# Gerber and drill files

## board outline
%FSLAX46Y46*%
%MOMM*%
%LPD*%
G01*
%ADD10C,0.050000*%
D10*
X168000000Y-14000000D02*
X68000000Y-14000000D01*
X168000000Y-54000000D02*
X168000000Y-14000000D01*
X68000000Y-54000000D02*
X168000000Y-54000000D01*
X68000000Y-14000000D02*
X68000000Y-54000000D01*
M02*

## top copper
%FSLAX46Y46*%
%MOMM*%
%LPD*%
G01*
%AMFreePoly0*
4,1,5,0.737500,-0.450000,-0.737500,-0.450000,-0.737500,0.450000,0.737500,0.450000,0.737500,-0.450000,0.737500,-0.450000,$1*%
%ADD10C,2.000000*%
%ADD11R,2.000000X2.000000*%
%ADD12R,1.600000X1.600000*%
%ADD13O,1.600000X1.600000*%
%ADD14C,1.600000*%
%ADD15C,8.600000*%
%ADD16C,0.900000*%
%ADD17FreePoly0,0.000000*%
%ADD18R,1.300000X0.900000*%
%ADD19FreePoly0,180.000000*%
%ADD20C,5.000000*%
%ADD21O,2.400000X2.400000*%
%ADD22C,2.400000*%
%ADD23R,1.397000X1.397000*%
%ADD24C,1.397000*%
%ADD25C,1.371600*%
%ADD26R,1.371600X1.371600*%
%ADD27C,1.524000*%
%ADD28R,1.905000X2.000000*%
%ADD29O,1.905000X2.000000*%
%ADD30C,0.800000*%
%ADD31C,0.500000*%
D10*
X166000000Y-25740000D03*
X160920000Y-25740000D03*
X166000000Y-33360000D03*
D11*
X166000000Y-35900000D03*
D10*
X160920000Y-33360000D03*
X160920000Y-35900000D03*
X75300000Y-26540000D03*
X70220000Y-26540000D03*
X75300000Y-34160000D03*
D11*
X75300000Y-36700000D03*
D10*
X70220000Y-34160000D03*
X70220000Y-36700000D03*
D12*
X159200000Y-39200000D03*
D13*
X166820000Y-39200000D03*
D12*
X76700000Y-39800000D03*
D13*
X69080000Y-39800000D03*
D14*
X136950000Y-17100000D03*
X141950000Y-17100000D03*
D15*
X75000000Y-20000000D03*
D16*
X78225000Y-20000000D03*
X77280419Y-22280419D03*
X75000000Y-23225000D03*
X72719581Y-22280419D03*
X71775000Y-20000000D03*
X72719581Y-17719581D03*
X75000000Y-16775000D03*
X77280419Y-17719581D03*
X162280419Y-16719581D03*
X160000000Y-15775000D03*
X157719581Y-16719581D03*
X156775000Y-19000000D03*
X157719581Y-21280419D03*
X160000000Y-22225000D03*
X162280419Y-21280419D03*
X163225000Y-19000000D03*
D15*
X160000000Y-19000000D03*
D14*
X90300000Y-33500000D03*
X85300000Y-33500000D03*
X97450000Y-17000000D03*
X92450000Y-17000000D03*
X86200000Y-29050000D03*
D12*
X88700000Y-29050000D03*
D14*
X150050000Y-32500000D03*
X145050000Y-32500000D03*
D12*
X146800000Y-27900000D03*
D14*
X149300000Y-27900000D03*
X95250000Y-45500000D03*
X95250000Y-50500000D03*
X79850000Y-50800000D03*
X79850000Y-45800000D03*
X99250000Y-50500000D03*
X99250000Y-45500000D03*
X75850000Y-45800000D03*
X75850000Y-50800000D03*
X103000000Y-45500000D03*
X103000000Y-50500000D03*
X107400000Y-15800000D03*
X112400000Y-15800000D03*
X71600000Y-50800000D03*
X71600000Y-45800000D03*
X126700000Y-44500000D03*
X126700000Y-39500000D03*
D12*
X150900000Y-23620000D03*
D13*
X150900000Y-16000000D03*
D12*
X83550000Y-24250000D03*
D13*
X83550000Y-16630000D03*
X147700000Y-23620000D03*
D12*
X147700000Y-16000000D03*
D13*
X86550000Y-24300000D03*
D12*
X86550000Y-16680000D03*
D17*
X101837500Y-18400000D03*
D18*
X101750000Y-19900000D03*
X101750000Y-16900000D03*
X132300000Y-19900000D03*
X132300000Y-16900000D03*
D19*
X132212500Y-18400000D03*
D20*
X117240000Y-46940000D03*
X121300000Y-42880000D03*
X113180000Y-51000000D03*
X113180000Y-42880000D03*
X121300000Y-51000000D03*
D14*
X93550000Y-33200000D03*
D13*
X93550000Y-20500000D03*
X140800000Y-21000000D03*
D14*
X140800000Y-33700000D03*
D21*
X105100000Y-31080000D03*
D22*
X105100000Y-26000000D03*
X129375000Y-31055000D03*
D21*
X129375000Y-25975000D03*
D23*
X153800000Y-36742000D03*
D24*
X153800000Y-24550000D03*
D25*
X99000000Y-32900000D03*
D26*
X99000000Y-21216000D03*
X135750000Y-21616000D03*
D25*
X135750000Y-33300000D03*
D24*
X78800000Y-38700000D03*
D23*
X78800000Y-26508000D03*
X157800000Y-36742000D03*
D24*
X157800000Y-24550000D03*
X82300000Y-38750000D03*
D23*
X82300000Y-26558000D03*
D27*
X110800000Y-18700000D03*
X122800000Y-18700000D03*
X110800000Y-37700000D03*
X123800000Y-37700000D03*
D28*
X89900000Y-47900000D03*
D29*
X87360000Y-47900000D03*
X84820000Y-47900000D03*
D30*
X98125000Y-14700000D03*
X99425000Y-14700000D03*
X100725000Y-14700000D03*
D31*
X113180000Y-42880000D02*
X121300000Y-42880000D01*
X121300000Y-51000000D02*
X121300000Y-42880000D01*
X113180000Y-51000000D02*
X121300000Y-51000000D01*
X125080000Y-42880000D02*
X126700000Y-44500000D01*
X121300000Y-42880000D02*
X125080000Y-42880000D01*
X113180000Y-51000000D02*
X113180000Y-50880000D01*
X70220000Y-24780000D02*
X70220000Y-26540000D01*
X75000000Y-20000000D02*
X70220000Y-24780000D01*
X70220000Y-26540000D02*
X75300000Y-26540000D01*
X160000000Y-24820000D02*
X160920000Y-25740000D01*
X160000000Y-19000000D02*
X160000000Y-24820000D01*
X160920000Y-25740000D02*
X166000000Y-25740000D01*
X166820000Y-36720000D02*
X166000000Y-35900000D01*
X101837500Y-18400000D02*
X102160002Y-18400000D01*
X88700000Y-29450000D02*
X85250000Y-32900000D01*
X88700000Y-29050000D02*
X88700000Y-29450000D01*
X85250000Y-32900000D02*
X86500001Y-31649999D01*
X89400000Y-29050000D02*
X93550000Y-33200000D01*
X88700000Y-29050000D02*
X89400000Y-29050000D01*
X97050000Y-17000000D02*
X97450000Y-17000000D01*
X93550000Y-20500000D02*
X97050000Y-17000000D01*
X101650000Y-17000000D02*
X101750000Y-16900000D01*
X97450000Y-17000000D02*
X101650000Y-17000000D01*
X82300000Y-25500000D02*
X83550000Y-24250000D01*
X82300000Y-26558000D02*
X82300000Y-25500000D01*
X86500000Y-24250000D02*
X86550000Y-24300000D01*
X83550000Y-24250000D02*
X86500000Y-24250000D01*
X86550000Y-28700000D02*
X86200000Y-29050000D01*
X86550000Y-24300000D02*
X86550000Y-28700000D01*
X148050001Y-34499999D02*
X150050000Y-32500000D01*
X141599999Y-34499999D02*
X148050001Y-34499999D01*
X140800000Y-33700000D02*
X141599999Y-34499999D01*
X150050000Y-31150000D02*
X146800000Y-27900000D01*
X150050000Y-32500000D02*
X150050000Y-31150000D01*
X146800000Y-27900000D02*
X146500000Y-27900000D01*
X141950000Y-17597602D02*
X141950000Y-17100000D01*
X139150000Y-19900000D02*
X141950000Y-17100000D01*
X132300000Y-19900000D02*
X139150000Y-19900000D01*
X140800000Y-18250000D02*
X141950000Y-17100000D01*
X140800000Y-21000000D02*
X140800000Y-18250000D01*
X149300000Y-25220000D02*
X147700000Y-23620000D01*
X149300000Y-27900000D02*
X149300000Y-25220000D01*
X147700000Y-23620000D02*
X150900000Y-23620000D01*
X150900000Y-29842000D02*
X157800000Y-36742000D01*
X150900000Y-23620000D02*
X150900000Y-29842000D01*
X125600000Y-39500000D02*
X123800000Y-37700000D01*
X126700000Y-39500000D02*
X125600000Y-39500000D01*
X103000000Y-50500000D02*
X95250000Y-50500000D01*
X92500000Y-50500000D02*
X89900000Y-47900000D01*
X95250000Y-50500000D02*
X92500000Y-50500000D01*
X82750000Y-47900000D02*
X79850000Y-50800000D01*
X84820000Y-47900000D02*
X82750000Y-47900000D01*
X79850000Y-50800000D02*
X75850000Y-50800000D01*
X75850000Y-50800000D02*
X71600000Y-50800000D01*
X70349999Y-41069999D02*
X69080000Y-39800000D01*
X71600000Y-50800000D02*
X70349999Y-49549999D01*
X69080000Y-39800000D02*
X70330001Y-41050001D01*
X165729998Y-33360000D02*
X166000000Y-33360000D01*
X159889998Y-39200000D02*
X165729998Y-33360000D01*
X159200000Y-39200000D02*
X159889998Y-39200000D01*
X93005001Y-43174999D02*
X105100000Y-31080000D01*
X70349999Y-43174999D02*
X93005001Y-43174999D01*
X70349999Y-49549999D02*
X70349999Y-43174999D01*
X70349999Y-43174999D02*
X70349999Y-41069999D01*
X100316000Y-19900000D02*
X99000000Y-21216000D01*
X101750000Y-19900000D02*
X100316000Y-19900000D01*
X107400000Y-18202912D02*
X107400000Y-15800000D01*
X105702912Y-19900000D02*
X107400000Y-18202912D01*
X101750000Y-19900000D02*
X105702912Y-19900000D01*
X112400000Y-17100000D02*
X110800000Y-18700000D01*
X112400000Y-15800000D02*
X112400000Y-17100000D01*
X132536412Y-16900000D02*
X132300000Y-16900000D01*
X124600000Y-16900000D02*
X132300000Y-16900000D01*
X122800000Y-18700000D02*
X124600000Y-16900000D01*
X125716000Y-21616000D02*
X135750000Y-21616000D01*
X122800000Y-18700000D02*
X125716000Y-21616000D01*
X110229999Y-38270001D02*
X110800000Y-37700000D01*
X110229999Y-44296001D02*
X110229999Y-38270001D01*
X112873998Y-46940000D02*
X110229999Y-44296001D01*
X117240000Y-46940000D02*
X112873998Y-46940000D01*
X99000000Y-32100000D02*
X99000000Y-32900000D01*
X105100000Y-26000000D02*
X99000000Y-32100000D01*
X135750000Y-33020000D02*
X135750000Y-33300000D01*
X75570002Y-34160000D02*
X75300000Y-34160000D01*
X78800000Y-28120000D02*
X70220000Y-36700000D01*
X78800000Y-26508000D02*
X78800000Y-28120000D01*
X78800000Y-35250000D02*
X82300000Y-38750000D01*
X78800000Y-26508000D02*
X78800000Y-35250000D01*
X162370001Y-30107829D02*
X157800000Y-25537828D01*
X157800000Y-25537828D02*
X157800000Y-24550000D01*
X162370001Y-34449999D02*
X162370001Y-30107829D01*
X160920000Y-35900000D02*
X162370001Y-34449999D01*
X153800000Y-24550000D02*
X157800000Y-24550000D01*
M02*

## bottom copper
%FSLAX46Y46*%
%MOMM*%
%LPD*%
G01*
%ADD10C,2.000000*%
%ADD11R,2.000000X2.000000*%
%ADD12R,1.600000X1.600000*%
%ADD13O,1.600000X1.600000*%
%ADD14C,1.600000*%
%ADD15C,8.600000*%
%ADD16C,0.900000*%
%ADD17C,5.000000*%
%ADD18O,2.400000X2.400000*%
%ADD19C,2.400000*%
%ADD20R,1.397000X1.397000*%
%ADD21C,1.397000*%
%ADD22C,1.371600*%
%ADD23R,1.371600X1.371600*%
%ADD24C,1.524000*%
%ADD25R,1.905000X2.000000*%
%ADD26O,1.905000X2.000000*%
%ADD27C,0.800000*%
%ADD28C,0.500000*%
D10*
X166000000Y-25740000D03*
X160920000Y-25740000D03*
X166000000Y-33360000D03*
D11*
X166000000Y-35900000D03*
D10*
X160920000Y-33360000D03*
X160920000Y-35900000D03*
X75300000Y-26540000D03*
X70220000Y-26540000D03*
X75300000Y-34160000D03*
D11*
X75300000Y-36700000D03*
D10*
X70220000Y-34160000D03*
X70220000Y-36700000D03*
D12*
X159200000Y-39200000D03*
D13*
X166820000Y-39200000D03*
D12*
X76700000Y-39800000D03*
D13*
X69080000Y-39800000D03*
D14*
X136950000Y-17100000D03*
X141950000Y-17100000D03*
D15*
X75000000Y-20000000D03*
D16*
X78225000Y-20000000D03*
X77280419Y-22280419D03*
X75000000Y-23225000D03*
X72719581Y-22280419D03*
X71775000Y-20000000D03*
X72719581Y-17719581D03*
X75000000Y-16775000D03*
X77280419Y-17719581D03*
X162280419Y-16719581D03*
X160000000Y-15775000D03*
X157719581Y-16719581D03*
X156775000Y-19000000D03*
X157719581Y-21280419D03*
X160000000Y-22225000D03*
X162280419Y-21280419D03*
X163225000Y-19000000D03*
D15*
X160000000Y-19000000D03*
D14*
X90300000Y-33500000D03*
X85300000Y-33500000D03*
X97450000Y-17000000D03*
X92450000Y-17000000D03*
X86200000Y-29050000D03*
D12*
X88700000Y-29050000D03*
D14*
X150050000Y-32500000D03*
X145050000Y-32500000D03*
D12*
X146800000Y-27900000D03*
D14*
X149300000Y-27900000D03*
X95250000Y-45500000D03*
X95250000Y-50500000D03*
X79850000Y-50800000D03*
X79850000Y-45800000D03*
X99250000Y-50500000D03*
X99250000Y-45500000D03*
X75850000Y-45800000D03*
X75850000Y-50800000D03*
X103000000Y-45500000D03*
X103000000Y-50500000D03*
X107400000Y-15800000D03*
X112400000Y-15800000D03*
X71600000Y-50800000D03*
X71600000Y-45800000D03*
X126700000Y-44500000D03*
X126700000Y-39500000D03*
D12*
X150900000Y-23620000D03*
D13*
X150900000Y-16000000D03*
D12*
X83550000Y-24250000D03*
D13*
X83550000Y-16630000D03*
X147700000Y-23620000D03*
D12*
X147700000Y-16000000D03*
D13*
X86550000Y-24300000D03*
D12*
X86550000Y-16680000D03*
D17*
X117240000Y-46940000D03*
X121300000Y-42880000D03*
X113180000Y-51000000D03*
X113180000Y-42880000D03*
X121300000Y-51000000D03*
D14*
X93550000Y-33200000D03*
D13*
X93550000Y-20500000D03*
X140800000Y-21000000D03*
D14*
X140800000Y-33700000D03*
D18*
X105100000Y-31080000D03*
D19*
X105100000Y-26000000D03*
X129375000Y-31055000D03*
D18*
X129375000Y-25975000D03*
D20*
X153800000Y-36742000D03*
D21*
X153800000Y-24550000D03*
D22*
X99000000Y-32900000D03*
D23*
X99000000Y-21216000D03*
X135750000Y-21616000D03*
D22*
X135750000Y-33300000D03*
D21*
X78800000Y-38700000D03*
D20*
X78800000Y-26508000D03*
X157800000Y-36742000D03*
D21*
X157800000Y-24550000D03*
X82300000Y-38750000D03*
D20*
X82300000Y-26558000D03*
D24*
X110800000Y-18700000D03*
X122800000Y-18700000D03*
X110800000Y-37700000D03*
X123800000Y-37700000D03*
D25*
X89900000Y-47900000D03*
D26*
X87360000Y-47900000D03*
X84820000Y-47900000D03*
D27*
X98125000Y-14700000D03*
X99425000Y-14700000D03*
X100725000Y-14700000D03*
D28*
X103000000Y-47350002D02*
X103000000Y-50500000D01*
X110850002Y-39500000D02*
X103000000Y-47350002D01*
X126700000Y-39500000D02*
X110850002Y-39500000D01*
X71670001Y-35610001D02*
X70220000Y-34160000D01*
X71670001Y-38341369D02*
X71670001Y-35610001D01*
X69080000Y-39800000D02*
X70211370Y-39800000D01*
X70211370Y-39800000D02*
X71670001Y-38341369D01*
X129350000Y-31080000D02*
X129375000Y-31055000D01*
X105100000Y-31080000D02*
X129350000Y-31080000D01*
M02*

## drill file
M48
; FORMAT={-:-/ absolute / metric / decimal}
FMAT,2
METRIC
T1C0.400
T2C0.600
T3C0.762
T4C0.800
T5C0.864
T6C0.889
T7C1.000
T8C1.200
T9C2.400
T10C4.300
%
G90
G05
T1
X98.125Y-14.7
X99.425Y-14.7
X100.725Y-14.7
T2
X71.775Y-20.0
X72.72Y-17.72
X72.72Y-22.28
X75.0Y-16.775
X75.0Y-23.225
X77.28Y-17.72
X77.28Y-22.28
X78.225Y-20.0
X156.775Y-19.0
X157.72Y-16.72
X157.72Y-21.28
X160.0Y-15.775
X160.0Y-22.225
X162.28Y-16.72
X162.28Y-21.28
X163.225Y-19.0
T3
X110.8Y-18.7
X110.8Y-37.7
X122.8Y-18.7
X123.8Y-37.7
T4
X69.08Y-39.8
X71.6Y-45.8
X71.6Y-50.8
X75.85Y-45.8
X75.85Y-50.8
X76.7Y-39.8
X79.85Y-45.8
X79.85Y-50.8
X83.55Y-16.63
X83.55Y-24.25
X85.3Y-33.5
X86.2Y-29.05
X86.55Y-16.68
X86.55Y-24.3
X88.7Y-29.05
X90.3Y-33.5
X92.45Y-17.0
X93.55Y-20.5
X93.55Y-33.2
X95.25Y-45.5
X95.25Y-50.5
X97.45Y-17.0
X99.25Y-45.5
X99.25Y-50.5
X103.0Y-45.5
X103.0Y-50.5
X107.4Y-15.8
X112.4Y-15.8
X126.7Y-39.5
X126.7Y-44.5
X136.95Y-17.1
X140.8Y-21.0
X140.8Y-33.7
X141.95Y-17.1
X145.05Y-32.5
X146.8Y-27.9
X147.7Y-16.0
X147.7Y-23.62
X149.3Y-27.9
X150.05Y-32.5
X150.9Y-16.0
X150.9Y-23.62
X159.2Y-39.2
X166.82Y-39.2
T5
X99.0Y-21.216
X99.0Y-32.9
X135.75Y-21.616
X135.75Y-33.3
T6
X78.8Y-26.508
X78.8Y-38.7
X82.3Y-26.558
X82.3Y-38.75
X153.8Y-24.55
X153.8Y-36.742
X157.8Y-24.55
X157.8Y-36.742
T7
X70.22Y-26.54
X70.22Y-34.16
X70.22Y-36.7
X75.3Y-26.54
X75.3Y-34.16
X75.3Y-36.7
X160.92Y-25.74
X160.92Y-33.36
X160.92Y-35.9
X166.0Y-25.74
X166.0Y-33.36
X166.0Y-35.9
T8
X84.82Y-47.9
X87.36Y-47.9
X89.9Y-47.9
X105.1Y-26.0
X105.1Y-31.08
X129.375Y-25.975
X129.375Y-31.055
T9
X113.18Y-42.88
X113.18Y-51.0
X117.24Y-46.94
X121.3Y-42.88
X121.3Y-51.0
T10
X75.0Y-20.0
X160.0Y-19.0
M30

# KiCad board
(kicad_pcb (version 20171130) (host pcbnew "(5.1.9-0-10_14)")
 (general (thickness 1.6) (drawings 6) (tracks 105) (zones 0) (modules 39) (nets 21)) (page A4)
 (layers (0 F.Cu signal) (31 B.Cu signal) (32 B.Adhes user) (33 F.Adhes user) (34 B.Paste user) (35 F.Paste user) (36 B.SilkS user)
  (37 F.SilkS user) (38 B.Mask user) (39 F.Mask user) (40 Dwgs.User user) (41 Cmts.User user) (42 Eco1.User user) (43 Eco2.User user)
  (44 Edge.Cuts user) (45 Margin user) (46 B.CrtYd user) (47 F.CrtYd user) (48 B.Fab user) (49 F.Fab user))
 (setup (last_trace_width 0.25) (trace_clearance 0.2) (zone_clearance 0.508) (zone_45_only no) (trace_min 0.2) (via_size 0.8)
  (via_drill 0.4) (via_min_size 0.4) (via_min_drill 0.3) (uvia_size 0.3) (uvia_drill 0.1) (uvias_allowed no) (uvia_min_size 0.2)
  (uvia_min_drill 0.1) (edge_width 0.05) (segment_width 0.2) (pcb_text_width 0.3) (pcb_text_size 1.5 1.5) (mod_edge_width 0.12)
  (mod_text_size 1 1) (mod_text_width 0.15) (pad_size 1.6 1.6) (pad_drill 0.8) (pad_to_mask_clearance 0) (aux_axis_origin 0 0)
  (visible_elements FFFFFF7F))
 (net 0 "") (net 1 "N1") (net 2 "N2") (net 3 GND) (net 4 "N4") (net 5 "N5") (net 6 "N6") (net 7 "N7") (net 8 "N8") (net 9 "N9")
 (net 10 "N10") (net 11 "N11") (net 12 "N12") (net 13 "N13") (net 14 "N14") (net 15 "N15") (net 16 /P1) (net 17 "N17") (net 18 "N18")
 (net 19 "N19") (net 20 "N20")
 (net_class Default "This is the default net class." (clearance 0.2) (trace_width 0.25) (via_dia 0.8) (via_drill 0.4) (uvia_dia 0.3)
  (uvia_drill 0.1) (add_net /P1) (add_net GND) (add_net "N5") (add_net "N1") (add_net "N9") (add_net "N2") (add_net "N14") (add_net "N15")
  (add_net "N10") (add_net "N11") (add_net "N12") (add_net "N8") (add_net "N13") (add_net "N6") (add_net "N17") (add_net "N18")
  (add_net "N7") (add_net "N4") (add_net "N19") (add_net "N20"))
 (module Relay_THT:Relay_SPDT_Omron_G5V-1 (layer F.Cu) (at 166 35.9 180)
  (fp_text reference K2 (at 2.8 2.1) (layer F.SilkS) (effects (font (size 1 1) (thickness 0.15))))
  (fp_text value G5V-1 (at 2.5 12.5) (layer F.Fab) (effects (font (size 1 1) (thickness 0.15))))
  (pad 5 thru_hole circle (at 0 10.16 180) (size 2 2) (drill 1) (layers *.Cu *.Mask) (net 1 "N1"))
  (pad 6 thru_hole circle (at 5.08 10.16 180) (size 2 2) (drill 1) (layers *.Cu *.Mask) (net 1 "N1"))
  (pad 2 thru_hole circle (at 0 2.54 180) (size 2 2) (drill 1) (layers *.Cu *.Mask) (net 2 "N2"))
  (pad 1 thru_hole rect (at 0 0 180) (size 2 2) (drill 1) (layers *.Cu *.Mask) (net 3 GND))
  (pad 9 thru_hole circle (at 5.08 2.54 180) (size 2 2) (drill 1) (layers *.Cu *.Mask) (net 3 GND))
  (pad 10 thru_hole circle (at 5.08 0 180) (size 2 2) (drill 1) (layers *.Cu *.Mask) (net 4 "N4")))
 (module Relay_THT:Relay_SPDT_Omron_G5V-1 (layer F.Cu) (at 75.3 36.7 180)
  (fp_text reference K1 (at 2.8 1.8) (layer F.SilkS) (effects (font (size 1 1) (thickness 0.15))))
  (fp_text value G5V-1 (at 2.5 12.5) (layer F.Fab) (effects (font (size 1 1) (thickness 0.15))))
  (pad 5 thru_hole circle (at 0 10.16 180) (size 2 2) (drill 1) (layers *.Cu *.Mask) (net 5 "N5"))
  (pad 6 thru_hole circle (at 5.08 10.16 180) (size 2 2) (drill 1) (layers *.Cu *.Mask) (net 5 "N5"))
  (pad 2 thru_hole circle (at 0 2.54 180) (size 2 2) (drill 1) (layers *.Cu *.Mask) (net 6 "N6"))
  (pad 1 thru_hole rect (at 0 0 180) (size 2 2) (drill 1) (layers *.Cu *.Mask) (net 3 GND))
  (pad 9 thru_hole circle (at 5.08 2.54 180) (size 2 2) (drill 1) (layers *.Cu *.Mask) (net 2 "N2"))
  (pad 10 thru_hole circle (at 5.08 0 180) (size 2 2) (drill 1) (layers *.Cu *.Mask) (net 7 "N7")))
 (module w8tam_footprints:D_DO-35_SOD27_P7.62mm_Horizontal (layer F.Cu) (at 159.2 39.2)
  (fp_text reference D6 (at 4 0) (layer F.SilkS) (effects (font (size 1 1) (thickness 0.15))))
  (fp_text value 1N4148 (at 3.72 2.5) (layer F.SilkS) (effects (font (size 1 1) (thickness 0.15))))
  (pad 1 thru_hole rect (at 0 0) (size 1.6 1.6) (drill 0.8) (layers *.Cu *.Mask) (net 2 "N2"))
  (pad 2 thru_hole oval (at 7.62 0) (size 1.6 1.6) (drill 0.8) (layers *.Cu *.Mask) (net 3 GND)))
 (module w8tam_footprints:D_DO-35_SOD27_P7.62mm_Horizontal (layer F.Cu) (at 76.7 39.8 180)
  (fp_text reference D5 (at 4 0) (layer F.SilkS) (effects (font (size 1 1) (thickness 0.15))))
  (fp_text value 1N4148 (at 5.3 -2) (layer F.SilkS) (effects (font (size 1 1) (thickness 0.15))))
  (pad 1 thru_hole rect (at 0 0 180) (size 1.6 1.6) (drill 0.8) (layers *.Cu *.Mask) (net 3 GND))
  (pad 2 thru_hole oval (at 7.62 0 180) (size 1.6 1.6) (drill 0.8) (layers *.Cu *.Mask) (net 2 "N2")))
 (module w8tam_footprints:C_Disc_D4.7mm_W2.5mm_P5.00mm (layer F.Cu) (at 141.95 17.1 180)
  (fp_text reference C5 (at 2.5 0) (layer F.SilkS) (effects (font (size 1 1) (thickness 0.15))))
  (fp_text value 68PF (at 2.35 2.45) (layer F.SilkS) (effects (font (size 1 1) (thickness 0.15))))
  (pad 2 thru_hole circle (at 5 0 180) (size 1.6 1.6) (drill 0.8) (layers *.Cu *.Mask) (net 3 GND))
  (pad 1 thru_hole circle (at 0 0 180) (size 1.6 1.6) (drill 0.8) (layers *.Cu *.Mask) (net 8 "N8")))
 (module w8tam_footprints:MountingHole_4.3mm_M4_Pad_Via (layer F.Cu) (at 75 20)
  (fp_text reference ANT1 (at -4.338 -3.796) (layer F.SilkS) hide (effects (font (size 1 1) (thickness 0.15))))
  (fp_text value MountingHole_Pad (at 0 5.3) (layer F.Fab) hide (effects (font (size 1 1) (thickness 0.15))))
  (pad 1 thru_hole circle (at 0 0) (size 8.6 8.6) (drill 4.3) (layers *.Cu *.Mask) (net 5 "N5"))
  (pad 1 thru_hole circle (at 3.225 0) (size 0.9 0.9) (drill 0.6) (layers *.Cu *.Mask) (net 5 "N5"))
  (pad 1 thru_hole circle (at 2.280419 2.280419) (size 0.9 0.9) (drill 0.6) (layers *.Cu *.Mask) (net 5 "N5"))
  (pad 1 thru_hole circle (at 0 3.225) (size 0.9 0.9) (drill 0.6) (layers *.Cu *.Mask) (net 5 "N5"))
  (pad 1 thru_hole circle (at -2.280419 2.280419) (size 0.9 0.9) (drill 0.6) (layers *.Cu *.Mask) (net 5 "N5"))
  (pad 1 thru_hole circle (at -3.225 0) (size 0.9 0.9) (drill 0.6) (layers *.Cu *.Mask) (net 5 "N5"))
  (pad 1 thru_hole circle (at -2.280419 -2.280419) (size 0.9 0.9) (drill 0.6) (layers *.Cu *.Mask) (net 5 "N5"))
  (pad 1 thru_hole circle (at 0 -3.225) (size 0.9 0.9) (drill 0.6) (layers *.Cu *.Mask) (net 5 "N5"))
  (pad 1 thru_hole circle (at 2.280419 -2.280419) (size 0.9 0.9) (drill 0.6) (layers *.Cu *.Mask) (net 5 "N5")))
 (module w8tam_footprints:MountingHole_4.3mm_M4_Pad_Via (layer F.Cu) (at 160 19)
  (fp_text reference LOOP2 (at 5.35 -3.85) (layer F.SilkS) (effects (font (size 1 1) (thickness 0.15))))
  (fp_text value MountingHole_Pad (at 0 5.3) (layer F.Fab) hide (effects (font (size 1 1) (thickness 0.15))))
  (pad 1 thru_hole circle (at 2.280419 -2.280419) (size 0.9 0.9) (drill 0.6) (layers *.Cu *.Mask) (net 1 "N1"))
  (pad 1 thru_hole circle (at 0 -3.225) (size 0.9 0.9) (drill 0.6) (layers *.Cu *.Mask) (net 1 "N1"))
  (pad 1 thru_hole circle (at -2.280419 -2.280419) (size 0.9 0.9) (drill 0.6) (layers *.Cu *.Mask) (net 1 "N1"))
  (pad 1 thru_hole circle (at -3.225 0) (size 0.9 0.9) (drill 0.6) (layers *.Cu *.Mask) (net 1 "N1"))
  (pad 1 thru_hole circle (at -2.280419 2.280419) (size 0.9 0.9) (drill 0.6) (layers *.Cu *.Mask) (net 1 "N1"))
  (pad 1 thru_hole circle (at 0 3.225) (size 0.9 0.9) (drill 0.6) (layers *.Cu *.Mask) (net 1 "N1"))
  (pad 1 thru_hole circle (at 2.280419 2.280419) (size 0.9 0.9) (drill 0.6) (layers *.Cu *.Mask) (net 1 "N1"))
  (pad 1 thru_hole circle (at 3.225 0) (size 0.9 0.9) (drill 0.6) (layers *.Cu *.Mask) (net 1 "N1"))
  (pad 1 thru_hole circle (at 0 0) (size 8.6 8.6) (drill 4.3) (layers *.Cu *.Mask) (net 1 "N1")))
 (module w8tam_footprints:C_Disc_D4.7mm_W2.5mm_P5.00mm (layer F.Cu) (at 85.3 33.5)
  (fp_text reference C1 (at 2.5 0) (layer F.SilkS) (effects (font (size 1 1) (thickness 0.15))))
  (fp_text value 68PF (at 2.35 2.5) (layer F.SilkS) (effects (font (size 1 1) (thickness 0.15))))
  (pad 2 thru_hole circle (at 5 0) (size 1.6 1.6) (drill 0.8) (layers *.Cu *.Mask) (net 3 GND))
  (pad 1 thru_hole circle (at 0 0) (size 1.6 1.6) (drill 0.8) (layers *.Cu *.Mask) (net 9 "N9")))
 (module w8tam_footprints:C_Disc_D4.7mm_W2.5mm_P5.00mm (layer F.Cu) (at 97.45 17 180)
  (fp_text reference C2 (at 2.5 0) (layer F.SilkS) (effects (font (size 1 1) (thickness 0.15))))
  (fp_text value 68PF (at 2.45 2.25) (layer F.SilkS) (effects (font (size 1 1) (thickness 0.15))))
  (pad 1 thru_hole circle (at 0 0 180) (size 1.6 1.6) (drill 0.8) (layers *.Cu *.Mask) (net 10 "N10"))
  (pad 2 thru_hole circle (at 5 0 180) (size 1.6 1.6) (drill 0.8) (layers *.Cu *.Mask) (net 3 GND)))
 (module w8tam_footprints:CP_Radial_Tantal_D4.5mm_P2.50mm (layer F.Cu) (at 88.7 29.05 180)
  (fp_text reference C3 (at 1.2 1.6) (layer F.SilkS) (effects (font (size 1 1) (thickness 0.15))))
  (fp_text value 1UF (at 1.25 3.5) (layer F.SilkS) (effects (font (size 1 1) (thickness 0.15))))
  (pad 2 thru_hole circle (at 2.5 0 180) (size 1.6 1.6) (drill 0.8) (layers *.Cu *.Mask) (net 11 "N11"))
  (pad 1 thru_hole rect (at 0 0 180) (size 1.6 1.6) (drill 0.8) (layers *.Cu *.Mask) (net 9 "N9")))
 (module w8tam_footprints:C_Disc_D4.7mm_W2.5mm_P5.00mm (layer F.Cu) (at 150.05 32.5 180)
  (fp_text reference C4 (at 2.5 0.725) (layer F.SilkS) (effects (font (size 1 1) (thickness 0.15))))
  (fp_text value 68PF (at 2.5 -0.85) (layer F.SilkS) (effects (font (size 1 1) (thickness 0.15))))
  (pad 1 thru_hole circle (at 0 0 180) (size 1.6 1.6) (drill 0.8) (layers *.Cu *.Mask) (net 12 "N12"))
  (pad 2 thru_hole circle (at 5 0 180) (size 1.6 1.6) (drill 0.8) (layers *.Cu *.Mask) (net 3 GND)))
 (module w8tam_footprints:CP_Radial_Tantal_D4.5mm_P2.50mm (layer F.Cu) (at 146.8 27.9)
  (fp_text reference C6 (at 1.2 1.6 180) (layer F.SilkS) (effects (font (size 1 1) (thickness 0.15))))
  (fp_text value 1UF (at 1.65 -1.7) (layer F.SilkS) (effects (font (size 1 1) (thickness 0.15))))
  (pad 1 thru_hole rect (at 0 0) (size 1.6 1.6) (drill 0.8) (layers *.Cu *.Mask) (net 12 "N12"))
  (pad 2 thru_hole circle (at 2.5 0) (size 1.6 1.6) (drill 0.8) (layers *.Cu *.Mask) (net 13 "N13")))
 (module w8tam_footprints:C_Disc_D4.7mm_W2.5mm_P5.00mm (layer F.Cu) (at 95.25 50.5 90)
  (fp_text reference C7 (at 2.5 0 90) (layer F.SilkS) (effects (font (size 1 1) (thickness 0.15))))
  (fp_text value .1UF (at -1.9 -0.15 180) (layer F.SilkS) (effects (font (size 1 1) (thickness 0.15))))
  (pad 2 thru_hole circle (at 5 0 90) (size 1.6 1.6) (drill 0.8) (layers *.Cu *.Mask) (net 3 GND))
  (pad 1 thru_hole circle (at 0 0 90) (size 1.6 1.6) (drill 0.8) (layers *.Cu *.Mask) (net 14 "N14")))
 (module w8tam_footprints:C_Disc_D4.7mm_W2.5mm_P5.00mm (layer F.Cu) (at 79.85 50.8 90)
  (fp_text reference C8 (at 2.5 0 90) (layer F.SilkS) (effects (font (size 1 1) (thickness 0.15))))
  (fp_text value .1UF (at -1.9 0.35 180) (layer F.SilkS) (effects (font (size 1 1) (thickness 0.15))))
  (pad 1 thru_hole circle (at 0 0 90) (size 1.6 1.6) (drill 0.8) (layers *.Cu *.Mask) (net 2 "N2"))
  (pad 2 thru_hole circle (at 5 0 90) (size 1.6 1.6) (drill 0.8) (layers *.Cu *.Mask) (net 3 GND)))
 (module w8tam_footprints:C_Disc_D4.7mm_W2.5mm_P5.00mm (layer F.Cu) (at 99.25 50.5 90)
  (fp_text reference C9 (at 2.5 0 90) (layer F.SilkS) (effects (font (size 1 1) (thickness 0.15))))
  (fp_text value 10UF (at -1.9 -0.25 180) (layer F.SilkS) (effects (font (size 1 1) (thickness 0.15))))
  (pad 1 thru_hole circle (at 0 0 90) (size 1.6 1.6) (drill 0.8) (layers *.Cu *.Mask) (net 14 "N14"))
  (pad 2 thru_hole circle (at 5 0 90) (size 1.6 1.6) (drill 0.8) (layers *.Cu *.Mask) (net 3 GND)))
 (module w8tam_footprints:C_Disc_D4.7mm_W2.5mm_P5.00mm (layer F.Cu) (at 75.85 50.8 90)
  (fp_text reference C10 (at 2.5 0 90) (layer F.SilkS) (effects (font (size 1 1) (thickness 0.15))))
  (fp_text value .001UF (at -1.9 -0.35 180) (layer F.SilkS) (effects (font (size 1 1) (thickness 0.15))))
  (pad 2 thru_hole circle (at 5 0 90) (size 1.6 1.6) (drill 0.8) (layers *.Cu *.Mask) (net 3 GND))
  (pad 1 thru_hole circle (at 0 0 90) (size 1.6 1.6) (drill 0.8) (layers *.Cu *.Mask) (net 2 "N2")))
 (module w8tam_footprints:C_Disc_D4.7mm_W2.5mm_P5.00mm (layer F.Cu) (at 103 50.5 90)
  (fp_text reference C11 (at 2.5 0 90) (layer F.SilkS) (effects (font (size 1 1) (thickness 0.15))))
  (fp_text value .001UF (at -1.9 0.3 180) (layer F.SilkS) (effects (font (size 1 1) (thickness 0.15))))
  (pad 2 thru_hole circle (at 5 0 90) (size 1.6 1.6) (drill 0.8) (layers *.Cu *.Mask) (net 3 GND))
  (pad 1 thru_hole circle (at 0 0 90) (size 1.6 1.6) (drill 0.8) (layers *.Cu *.Mask) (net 14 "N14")))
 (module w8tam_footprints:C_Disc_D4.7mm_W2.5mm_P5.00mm (layer F.Cu) (at 112.4 15.8 180)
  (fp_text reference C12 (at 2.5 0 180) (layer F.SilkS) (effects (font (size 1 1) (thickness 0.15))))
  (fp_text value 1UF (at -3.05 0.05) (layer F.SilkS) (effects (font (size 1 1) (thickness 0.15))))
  (pad 2 thru_hole circle (at 5 0 180) (size 1.6 1.6) (drill 0.8) (layers *.Cu *.Mask) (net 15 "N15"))
  (pad 1 thru_hole circle (at 0 0 180) (size 1.6 1.6) (drill 0.8) (layers *.Cu *.Mask) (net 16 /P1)))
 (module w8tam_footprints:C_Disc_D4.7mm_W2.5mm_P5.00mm (layer F.Cu) (at 71.6 50.8 90)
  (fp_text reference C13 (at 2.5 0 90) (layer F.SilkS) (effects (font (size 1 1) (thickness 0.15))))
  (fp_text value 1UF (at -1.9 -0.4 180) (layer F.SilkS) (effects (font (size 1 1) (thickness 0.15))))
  (pad 1 thru_hole circle (at 0 0 90) (size 1.6 1.6) (drill 0.8) (layers *.Cu *.Mask) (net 2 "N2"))
  (pad 2 thru_hole circle (at 5 0 90) (size 1.6 1.6) (drill 0.8) (layers *.Cu *.Mask) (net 3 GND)))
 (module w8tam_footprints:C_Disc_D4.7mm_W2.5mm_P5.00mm (layer F.Cu) (at 126.7 44.5 90)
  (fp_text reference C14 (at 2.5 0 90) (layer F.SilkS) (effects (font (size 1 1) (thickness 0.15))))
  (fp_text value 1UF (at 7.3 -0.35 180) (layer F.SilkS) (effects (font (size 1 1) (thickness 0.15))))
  (pad 1 thru_hole circle (at 0 0 90) (size 1.6 1.6) (drill 0.8) (layers *.Cu *.Mask) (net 3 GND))
  (pad 2 thru_hole circle (at 5 0 90) (size 1.6 1.6) (drill 0.8) (layers *.Cu *.Mask) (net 14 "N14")))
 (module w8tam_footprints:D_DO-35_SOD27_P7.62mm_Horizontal (layer F.Cu) (at 150.9 23.62 90)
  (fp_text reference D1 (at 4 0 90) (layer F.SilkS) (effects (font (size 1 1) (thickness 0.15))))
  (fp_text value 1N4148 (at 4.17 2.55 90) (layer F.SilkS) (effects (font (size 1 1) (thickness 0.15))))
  (pad 1 thru_hole rect (at 0 0 90) (size 1.6 1.6) (drill 0.8) (layers *.Cu *.Mask) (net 13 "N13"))
  (pad 2 thru_hole oval (at 7.62 0 90) (size 1.6 1.6) (drill 0.8) (layers *.Cu *.Mask) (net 3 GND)))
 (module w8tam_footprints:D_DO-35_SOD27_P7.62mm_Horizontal (layer F.Cu) (at 83.55 24.25 90)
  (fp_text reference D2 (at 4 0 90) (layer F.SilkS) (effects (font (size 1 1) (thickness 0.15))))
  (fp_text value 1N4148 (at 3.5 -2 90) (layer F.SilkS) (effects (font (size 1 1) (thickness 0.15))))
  (pad 1 thru_hole rect (at 0 0 90) (size 1.6 1.6) (drill 0.8) (layers *.Cu *.Mask) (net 11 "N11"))
  (pad 2 thru_hole oval (at 7.62 0 90) (size 1.6 1.6) (drill 0.8) (layers *.Cu *.Mask) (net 3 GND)))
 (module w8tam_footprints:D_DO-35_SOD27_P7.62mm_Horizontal (layer F.Cu) (at 147.7 16 270)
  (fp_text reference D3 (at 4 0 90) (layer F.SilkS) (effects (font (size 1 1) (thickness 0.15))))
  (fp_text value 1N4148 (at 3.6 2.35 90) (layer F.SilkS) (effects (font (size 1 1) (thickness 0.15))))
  (pad 2 thru_hole oval (at 7.62 0 270) (size 1.6 1.6) (drill 0.8) (layers *.Cu *.Mask) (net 13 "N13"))
  (pad 1 thru_hole rect (at 0 0 270) (size 1.6 1.6) (drill 0.8) (layers *.Cu *.Mask) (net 3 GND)))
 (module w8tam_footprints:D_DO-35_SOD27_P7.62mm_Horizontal (layer F.Cu) (at 86.55 16.68 270)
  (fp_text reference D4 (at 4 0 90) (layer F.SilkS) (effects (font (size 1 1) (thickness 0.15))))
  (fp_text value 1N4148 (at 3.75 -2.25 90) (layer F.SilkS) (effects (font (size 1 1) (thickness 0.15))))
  (pad 2 thru_hole oval (at 7.62 0 270) (size 1.6 1.6) (drill 0.8) (layers *.Cu *.Mask) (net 11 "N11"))
  (pad 1 thru_hole rect (at 0 0 270) (size 1.6 1.6) (drill 0.8) (layers *.Cu *.Mask) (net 3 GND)))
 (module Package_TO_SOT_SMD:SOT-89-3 (layer F.Cu) (at 103.4 18.4)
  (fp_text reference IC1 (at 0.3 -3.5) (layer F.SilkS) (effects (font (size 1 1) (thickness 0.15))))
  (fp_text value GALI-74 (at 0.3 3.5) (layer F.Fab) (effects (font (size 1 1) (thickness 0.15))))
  (pad 2 smd custom (at -1.5625 0) (size 1.475 0.9) (layers F.Cu F.Paste F.Mask) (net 3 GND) (zone_connect 2)
   (options (clearance outline) (anchor rect)) (primitives))
  (pad 3 smd rect (at -1.65 1.5) (size 1.3 0.9) (layers F.Cu F.Paste F.Mask) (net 15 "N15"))
  (pad 1 smd rect (at -1.65 -1.5) (size 1.3 0.9) (layers F.Cu F.Paste F.Mask) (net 10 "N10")))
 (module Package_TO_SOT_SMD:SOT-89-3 (layer F.Cu) (at 130.65 18.4 180)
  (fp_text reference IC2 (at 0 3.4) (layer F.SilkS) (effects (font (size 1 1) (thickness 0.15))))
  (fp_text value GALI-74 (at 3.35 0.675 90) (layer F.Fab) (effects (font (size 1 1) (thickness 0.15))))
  (pad 1 smd rect (at -1.65 -1.5 180) (size 1.3 0.9) (layers F.Cu F.Paste F.Mask) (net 8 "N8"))
  (pad 3 smd rect (at -1.65 1.5 180) (size 1.3 0.9) (layers F.Cu F.Paste F.Mask) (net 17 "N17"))
  (pad 2 smd custom (at -1.5625 0 180) (size 1.475 0.9) (layers F.Cu F.Paste F.Mask) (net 3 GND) (zone_connect 2)
   (options (clearance outline) (anchor rect)) (primitives)))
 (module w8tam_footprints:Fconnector (layer B.Cu) (at 117.24 46.94)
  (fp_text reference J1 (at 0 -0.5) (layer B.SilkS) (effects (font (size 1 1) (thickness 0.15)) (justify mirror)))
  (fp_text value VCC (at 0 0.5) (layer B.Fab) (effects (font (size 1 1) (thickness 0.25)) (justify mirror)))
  (pad 1 thru_hole circle (at 0 0) (size 5 5) (drill 2.4) (layers *.Cu *.Mask) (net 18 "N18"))
  (pad 2 thru_hole circle (at 4.06 -4.06) (size 5 5) (drill 2.4) (layers *.Cu *.Mask) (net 3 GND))
  (pad 2 thru_hole circle (at -4.06 4.06) (size 5 5) (drill 2.4) (layers *.Cu *.Mask) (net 3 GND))
  (pad 2 thru_hole circle (at -4.06 -4.06) (size 5 5) (drill 2.4) (layers *.Cu *.Mask) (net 3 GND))
  (pad 2 thru_hole circle (at 4.06 4.06) (size 5 5) (drill 2.4) (layers *.Cu *.Mask) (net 3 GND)))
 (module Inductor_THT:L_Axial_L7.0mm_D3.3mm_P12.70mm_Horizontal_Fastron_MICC (layer F.Cu) (at 93.55 33.2 90)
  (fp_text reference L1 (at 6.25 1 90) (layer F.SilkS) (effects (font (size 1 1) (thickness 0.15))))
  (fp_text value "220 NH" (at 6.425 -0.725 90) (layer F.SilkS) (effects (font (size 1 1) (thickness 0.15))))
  (pad 1 thru_hole circle (at 0 0 90) (size 1.6 1.6) (drill 0.8) (layers *.Cu *.Mask) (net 9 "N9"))
  (pad 2 thru_hole oval (at 12.7 0 90) (size 1.6 1.6) (drill 0.8) (layers *.Cu *.Mask) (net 10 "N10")))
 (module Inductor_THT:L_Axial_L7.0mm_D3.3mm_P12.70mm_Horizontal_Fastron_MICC (layer F.Cu) (at 140.8 33.7 90)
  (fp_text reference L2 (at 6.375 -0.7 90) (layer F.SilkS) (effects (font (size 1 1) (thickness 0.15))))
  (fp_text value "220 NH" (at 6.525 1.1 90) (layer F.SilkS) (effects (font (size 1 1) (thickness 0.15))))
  (pad 2 thru_hole oval (at 12.7 0 90) (size 1.6 1.6) (drill 0.8) (layers *.Cu *.Mask) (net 8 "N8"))
  (pad 1 thru_hole circle (at 0 0 90) (size 1.6 1.6) (drill 0.8) (layers *.Cu *.Mask) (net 12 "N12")))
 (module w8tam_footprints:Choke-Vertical (layer F.Cu) (at 105.1 26 270)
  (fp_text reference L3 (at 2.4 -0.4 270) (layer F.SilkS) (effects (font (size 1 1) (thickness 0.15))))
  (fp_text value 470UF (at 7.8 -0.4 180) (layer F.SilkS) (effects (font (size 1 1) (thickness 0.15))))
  (pad 1 thru_hole oval (at 5.08 0 270) (size 2.4 2.4) (drill 1.2) (layers *.Cu *.Mask) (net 2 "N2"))
  (pad 2 thru_hole circle (at 0 0 270) (size 2.4 2.4) (drill 1.2) (layers *.Cu *.Mask) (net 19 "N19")))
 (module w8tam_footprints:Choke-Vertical (layer F.Cu) (at 129.375 31.055 90)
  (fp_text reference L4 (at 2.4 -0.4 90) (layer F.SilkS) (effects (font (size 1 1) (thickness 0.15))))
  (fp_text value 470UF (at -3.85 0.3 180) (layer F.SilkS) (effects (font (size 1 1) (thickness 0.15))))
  (pad 2 thru_hole circle (at 0 0 90) (size 2.4 2.4) (drill 1.2) (layers *.Cu *.Mask) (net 2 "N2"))
  (pad 1 thru_hole oval (at 5.08 0 90) (size 2.4 2.4) (drill 1.2) (layers *.Cu *.Mask) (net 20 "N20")))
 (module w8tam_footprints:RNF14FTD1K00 (layer F.Cu) (at 153.8 24.55 90)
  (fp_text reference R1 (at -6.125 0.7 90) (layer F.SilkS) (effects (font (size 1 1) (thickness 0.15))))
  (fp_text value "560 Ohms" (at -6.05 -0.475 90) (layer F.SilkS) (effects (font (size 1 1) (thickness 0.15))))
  (pad 1 thru_hole rect (at -12.192 0 90) (size 1.397 1.397) (drill 0.889) (layers *.Cu *.Mask) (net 3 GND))
  (pad 2 thru_hole circle (at 0 0 90) (size 1.397 1.397) (drill 0.889) (layers *.Cu *.Mask) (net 4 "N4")))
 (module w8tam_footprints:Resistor (layer F.Cu) (at 99 32.9 270)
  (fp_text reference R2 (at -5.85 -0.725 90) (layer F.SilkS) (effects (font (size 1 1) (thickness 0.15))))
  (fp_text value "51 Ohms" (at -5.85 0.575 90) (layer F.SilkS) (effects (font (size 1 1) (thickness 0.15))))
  (pad 2 thru_hole circle (at 0 0 270) (size 1.3716 1.3716) (drill 0.8636) (layers *.Cu *.Mask) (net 19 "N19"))
  (pad 1 thru_hole rect (at -11.684 0 270) (size 1.3716 1.3716) (drill 0.8636) (layers *.Cu *.Mask) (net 15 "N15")))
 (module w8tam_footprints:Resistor (layer F.Cu) (at 135.75 33.3 270)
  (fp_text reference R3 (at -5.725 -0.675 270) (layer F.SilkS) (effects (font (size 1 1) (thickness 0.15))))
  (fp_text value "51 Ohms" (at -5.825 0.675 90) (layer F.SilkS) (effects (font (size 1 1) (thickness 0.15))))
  (pad 1 thru_hole rect (at -11.684 0 270) (size 1.3716 1.3716) (drill 0.8636) (layers *.Cu *.Mask) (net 17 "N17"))
  (pad 2 thru_hole circle (at 0 0 270) (size 1.3716 1.3716) (drill 0.8636) (layers *.Cu *.Mask) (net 20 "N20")))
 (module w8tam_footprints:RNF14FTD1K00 (layer F.Cu) (at 78.8 38.7 270)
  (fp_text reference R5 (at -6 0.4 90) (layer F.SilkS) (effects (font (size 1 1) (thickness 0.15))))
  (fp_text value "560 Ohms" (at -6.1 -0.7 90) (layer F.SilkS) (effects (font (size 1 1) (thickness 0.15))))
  (pad 2 thru_hole circle (at 0 0 270) (size 1.397 1.397) (drill 0.889) (layers *.Cu *.Mask) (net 3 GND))
  (pad 1 thru_hole rect (at -12.192 0 270) (size 1.397 1.397) (drill 0.889) (layers *.Cu *.Mask) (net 7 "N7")))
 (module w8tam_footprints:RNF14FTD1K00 (layer F.Cu) (at 157.8 24.55 90)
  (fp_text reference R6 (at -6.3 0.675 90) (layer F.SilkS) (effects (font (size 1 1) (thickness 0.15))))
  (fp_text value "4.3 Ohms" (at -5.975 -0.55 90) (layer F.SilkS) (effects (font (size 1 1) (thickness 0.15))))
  (pad 1 thru_hole rect (at -12.192 0 90) (size 1.397 1.397) (drill 0.889) (layers *.Cu *.Mask) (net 13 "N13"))
  (pad 2 thru_hole circle (at 0 0 90) (size 1.397 1.397) (drill 0.889) (layers *.Cu *.Mask) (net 4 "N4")))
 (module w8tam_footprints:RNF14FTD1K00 (layer F.Cu) (at 82.3 38.75 270)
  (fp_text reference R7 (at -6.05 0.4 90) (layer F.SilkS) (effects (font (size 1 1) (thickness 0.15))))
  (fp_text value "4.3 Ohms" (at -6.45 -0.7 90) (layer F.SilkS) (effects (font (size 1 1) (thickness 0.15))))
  (pad 2 thru_hole circle (at 0 0 270) (size 1.397 1.397) (drill 0.889) (layers *.Cu *.Mask) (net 7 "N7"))
  (pad 1 thru_hole rect (at -12.192 0 270) (size 1.397 1.397) (drill 0.889) (layers *.Cu *.Mask) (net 11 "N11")))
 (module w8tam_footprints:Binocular (layer F.Cu) (at 118.8 34.7)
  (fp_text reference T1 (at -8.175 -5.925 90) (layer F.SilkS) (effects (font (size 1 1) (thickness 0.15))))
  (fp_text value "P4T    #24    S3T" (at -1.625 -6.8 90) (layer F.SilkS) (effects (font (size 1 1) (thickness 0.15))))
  (pad 1 thru_hole circle (at -8 -16) (size 1.524 1.524) (drill 0.762) (layers *.Cu *.Mask) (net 16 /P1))
  (pad 2 thru_hole circle (at 4 -16) (size 1.524 1.524) (drill 0.762) (layers *.Cu *.Mask) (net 17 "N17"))
  (pad 3 thru_hole circle (at -8 3) (size 1.524 1.524) (drill 0.762) (layers *.Cu *.Mask) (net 18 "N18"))
  (pad 4 thru_hole circle (at 5 3) (size 1.524 1.524) (drill 0.762) (layers *.Cu *.Mask) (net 14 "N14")))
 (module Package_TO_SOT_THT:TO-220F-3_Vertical (layer F.Cu) (at 89.9 47.9 180)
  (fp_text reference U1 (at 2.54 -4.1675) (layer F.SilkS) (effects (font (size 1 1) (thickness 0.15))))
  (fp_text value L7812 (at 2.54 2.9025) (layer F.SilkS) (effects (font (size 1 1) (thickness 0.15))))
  (pad 1 thru_hole rect (at 0 0 180) (size 1.905 2) (drill 1.2) (layers *.Cu *.Mask) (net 14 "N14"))
  (pad 2 thru_hole oval (at 2.54 0 180) (size 1.905 2) (drill 1.2) (layers *.Cu *.Mask) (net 3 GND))
  (pad 3 thru_hole oval (at 5.08 0 180) (size 1.905 2) (drill 1.2) (layers *.Cu *.Mask) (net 2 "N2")))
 (gr_line (start 168 14) (end 68 14) (layer Edge.Cuts) (width 0.05))
 (gr_line (start 168 54) (end 168 14) (layer Edge.Cuts) (width 0.05))
 (gr_line (start 68 54) (end 168 54) (layer Edge.Cuts) (width 0.05))
 (gr_line (start 68 14) (end 68 54) (layer Edge.Cuts) (width 0.05))
 (via (at 98.125 14.7) (size 0.8) (drill 0.4) (layers F.Cu B.Cu) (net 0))
 (via (at 99.425 14.7) (size 0.8) (drill 0.4) (layers F.Cu B.Cu) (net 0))
 (via (at 100.725 14.7) (size 0.8) (drill 0.4) (layers F.Cu B.Cu) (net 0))
 (segment (start 113.18 42.88) (end 121.3 42.88) (width 0.5) (layer F.Cu) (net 3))
 (segment (start 121.3 51) (end 121.3 42.88) (width 0.5) (layer F.Cu) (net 3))
 (segment (start 113.18 51) (end 121.3 51) (width 0.5) (layer F.Cu) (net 3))
 (segment (start 125.08 42.88) (end 126.7 44.5) (width 0.5) (layer F.Cu) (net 3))
 (segment (start 121.3 42.88) (end 125.08 42.88) (width 0.5) (layer F.Cu) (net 3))
 (segment (start 113.18 51) (end 113.18 50.88) (width 0.5) (layer F.Cu) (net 3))
 (segment (start 70.22 24.78) (end 70.22 26.54) (width 0.5) (layer F.Cu) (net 5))
 (segment (start 75 20) (end 70.22 24.78) (width 0.5) (layer F.Cu) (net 5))
 (segment (start 70.22 26.54) (end 75.3 26.54) (width 0.5) (layer F.Cu) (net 5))
 (segment (start 160 24.82) (end 160.92 25.74) (width 0.5) (layer F.Cu) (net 1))
 (segment (start 160 19) (end 160 24.82) (width 0.5) (layer F.Cu) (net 1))
 (segment (start 160.92 25.74) (end 166 25.74) (width 0.5) (layer F.Cu) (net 1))
 (segment (start 166.82 36.72) (end 166 35.9) (width 0.5) (layer F.Cu) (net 3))
 (segment (start 101.8375 18.4) (end 102.160002 18.4) (width 0.5) (layer F.Cu) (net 3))
 (segment (start 88.7 29.45) (end 85.25 32.9) (width 0.5) (layer F.Cu) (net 9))
 (segment (start 88.7 29.05) (end 88.7 29.45) (width 0.5) (layer F.Cu) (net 9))
 (segment (start 85.25 32.9) (end 86.500001 31.649999) (width 0.5) (layer F.Cu) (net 9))
 (segment (start 89.4 29.05) (end 93.55 33.2) (width 0.5) (layer F.Cu) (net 9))
 (segment (start 88.7 29.05) (end 89.4 29.05) (width 0.5) (layer F.Cu) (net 9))
 (segment (start 97.05 17) (end 97.45 17) (width 0.5) (layer F.Cu) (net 10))
 (segment (start 93.55 20.5) (end 97.05 17) (width 0.5) (layer F.Cu) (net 10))
 (segment (start 101.65 17) (end 101.75 16.9) (width 0.5) (layer F.Cu) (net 10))
 (segment (start 97.45 17) (end 101.65 17) (width 0.5) (layer F.Cu) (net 10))
 (segment (start 82.3 25.5) (end 83.55 24.25) (width 0.5) (layer F.Cu) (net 11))
 (segment (start 82.3 26.558) (end 82.3 25.5) (width 0.5) (layer F.Cu) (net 11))
 (segment (start 86.5 24.25) (end 86.55 24.3) (width 0.5) (layer F.Cu) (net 11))
 (segment (start 83.55 24.25) (end 86.5 24.25) (width 0.5) (layer F.Cu) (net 11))
 (segment (start 86.55 28.7) (end 86.2 29.05) (width 0.5) (layer F.Cu) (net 11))
 (segment (start 86.55 24.3) (end 86.55 28.7) (width 0.5) (layer F.Cu) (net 11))
 (segment (start 148.050001 34.499999) (end 150.05 32.5) (width 0.5) (layer F.Cu) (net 12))
 (segment (start 141.599999 34.499999) (end 148.050001 34.499999) (width 0.5) (layer F.Cu) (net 12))
 (segment (start 140.8 33.7) (end 141.599999 34.499999) (width 0.5) (layer F.Cu) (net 12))
 (segment (start 150.05 31.15) (end 146.8 27.9) (width 0.5) (layer F.Cu) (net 12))
 (segment (start 150.05 32.5) (end 150.05 31.15) (width 0.5) (layer F.Cu) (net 12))
 (segment (start 146.8 27.9) (end 146.5 27.9) (width 0.5) (layer F.Cu) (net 12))
 (segment (start 141.95 17.597602) (end 141.95 17.1) (width 0.5) (layer F.Cu) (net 8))
 (segment (start 139.15 19.9) (end 141.95 17.1) (width 0.5) (layer F.Cu) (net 8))
 (segment (start 132.3 19.9) (end 139.15 19.9) (width 0.5) (layer F.Cu) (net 8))
 (segment (start 140.8 18.25) (end 141.95 17.1) (width 0.5) (layer F.Cu) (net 8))
 (segment (start 140.8 21) (end 140.8 18.25) (width 0.5) (layer F.Cu) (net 8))
 (segment (start 149.3 25.22) (end 147.7 23.62) (width 0.5) (layer F.Cu) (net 13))
 (segment (start 149.3 27.9) (end 149.3 25.22) (width 0.5) (layer F.Cu) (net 13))
 (segment (start 147.7 23.62) (end 150.9 23.62) (width 0.5) (layer F.Cu) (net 13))
 (segment (start 150.9 29.842) (end 157.8 36.742) (width 0.5) (layer F.Cu) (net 13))
 (segment (start 150.9 23.62) (end 150.9 29.842) (width 0.5) (layer F.Cu) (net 13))
 (segment (start 125.6 39.5) (end 123.8 37.7) (width 0.5) (layer F.Cu) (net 14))
 (segment (start 126.7 39.5) (end 125.6 39.5) (width 0.5) (layer F.Cu) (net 14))
 (segment (start 103 47.350002) (end 103 50.5) (width 0.5) (layer B.Cu) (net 14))
 (segment (start 110.850002 39.5) (end 103 47.350002) (width 0.5) (layer B.Cu) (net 14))
 (segment (start 126.7 39.5) (end 110.850002 39.5) (width 0.5) (layer B.Cu) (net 14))
 (segment (start 103 50.5) (end 95.25 50.5) (width 0.5) (layer F.Cu) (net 14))
 (segment (start 92.5 50.5) (end 89.9 47.9) (width 0.5) (layer F.Cu) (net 14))
 (segment (start 95.25 50.5) (end 92.5 50.5) (width 0.5) (layer F.Cu) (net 14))
 (segment (start 82.75 47.9) (end 79.85 50.8) (width 0.5) (layer F.Cu) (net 2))
 (segment (start 84.82 47.9) (end 82.75 47.9) (width 0.5) (layer F.Cu) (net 2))
 (segment (start 79.85 50.8) (end 75.85 50.8) (width 0.5) (layer F.Cu) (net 2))
 (segment (start 75.85 50.8) (end 71.6 50.8) (width 0.5) (layer F.Cu) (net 2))
 (segment (start 70.349999 41.069999) (end 69.08 39.8) (width 0.5) (layer F.Cu) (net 2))
 (segment (start 71.6 50.8) (end 70.349999 49.549999) (width 0.5) (layer F.Cu) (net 2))
 (segment (start 69.08 39.8) (end 70.330001 41.050001) (width 0.5) (layer F.Cu) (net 2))
 (segment (start 165.729998 33.36) (end 166 33.36) (width 0.5) (layer F.Cu) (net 2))
 (segment (start 159.889998 39.2) (end 165.729998 33.36) (width 0.5) (layer F.Cu) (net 2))
 (segment (start 159.2 39.2) (end 159.889998 39.2) (width 0.5) (layer F.Cu) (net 2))
 (segment (start 71.670001 35.610001) (end 70.22 34.16) (width 0.5) (layer B.Cu) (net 2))
 (segment (start 71.670001 38.341369) (end 71.670001 35.610001) (width 0.5) (layer B.Cu) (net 2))
 (segment (start 69.08 39.8) (end 70.21137 39.8) (width 0.5) (layer B.Cu) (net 2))
 (segment (start 70.21137 39.8) (end 71.670001 38.341369) (width 0.5) (layer B.Cu) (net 2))
 (segment (start 93.005001 43.174999) (end 105.1 31.08) (width 0.5) (layer F.Cu) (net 2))
 (segment (start 70.349999 43.174999) (end 93.005001 43.174999) (width 0.5) (layer F.Cu) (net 2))
 (segment (start 70.349999 49.549999) (end 70.349999 43.174999) (width 0.5) (layer F.Cu) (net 2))
 (segment (start 70.349999 43.174999) (end 70.349999 41.069999) (width 0.5) (layer F.Cu) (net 2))
 (segment (start 129.35 31.08) (end 129.375 31.055) (width 0.5) (layer B.Cu) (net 2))
 (segment (start 105.1 31.08) (end 129.35 31.08) (width 0.5) (layer B.Cu) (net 2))
 (segment (start 100.316 19.9) (end 99 21.216) (width 0.5) (layer F.Cu) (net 15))
 (segment (start 101.75 19.9) (end 100.316 19.9) (width 0.5) (layer F.Cu) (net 15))
 (segment (start 107.4 18.202912) (end 107.4 15.8) (width 0.5) (layer F.Cu) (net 15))
 (segment (start 105.702912 19.9) (end 107.4 18.202912) (width 0.5) (layer F.Cu) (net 15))
 (segment (start 101.75 19.9) (end 105.702912 19.9) (width 0.5) (layer F.Cu) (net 15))
 (segment (start 112.4 17.1) (end 110.8 18.7) (width 0.5) (layer F.Cu) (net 16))
 (segment (start 112.4 15.8) (end 112.4 17.1) (width 0.5) (layer F.Cu) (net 16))
 (segment (start 132.536412 16.9) (end 132.3 16.9) (width 0.5) (layer F.Cu) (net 17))
 (segment (start 124.6 16.9) (end 132.3 16.9) (width 0.5) (layer F.Cu) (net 17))
 (segment (start 122.8 18.7) (end 124.6 16.9) (width 0.5) (layer F.Cu) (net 17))
 (segment (start 125.716 21.616) (end 135.75 21.616) (width 0.5) (layer F.Cu) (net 17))
 (segment (start 122.8 18.7) (end 125.716 21.616) (width 0.5) (layer F.Cu) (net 17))
 (segment (start 110.229999 38.270001) (end 110.8 37.7) (width 0.5) (layer F.Cu) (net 18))
 (segment (start 110.229999 44.296001) (end 110.229999 38.270001) (width 0.5) (layer F.Cu) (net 18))
 (segment (start 112.873998 46.94) (end 110.229999 44.296001) (width 0.5) (layer F.Cu) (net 18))
 (segment (start 117.24 46.94) (end 112.873998 46.94) (width 0.5) (layer F.Cu) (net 18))
 (segment (start 99 32.1) (end 99 32.9) (width 0.5) (layer F.Cu) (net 19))
 (segment (start 105.1 26) (end 99 32.1) (width 0.5) (layer F.Cu) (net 19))
 (segment (start 135.75 33.02) (end 135.75 33.3) (width 0.5) (layer F.Cu) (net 20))
 (segment (start 75.570002 34.16) (end 75.3 34.16) (width 0.5) (layer F.Cu) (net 6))
 (segment (start 78.8 28.12) (end 70.22 36.7) (width 0.5) (layer F.Cu) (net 7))
 (segment (start 78.8 26.508) (end 78.8 28.12) (width 0.5) (layer F.Cu) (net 7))
 (segment (start 78.8 35.25) (end 82.3 38.75) (width 0.5) (layer F.Cu) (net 7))
 (segment (start 78.8 26.508) (end 78.8 35.25) (width 0.5) (layer F.Cu) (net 7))
 (segment (start 162.370001 30.107829) (end 157.8 25.537828) (width 0.5) (layer F.Cu) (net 4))
 (segment (start 157.8 25.537828) (end 157.8 24.55) (width 0.5) (layer F.Cu) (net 4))
 (segment (start 162.370001 34.449999) (end 162.370001 30.107829) (width 0.5) (layer F.Cu) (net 4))
 (segment (start 160.92 35.9) (end 162.370001 34.449999) (width 0.5) (layer F.Cu) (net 4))
 (segment (start 153.8 24.55) (end 157.8 24.55) (width 0.5) (layer F.Cu) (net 4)))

